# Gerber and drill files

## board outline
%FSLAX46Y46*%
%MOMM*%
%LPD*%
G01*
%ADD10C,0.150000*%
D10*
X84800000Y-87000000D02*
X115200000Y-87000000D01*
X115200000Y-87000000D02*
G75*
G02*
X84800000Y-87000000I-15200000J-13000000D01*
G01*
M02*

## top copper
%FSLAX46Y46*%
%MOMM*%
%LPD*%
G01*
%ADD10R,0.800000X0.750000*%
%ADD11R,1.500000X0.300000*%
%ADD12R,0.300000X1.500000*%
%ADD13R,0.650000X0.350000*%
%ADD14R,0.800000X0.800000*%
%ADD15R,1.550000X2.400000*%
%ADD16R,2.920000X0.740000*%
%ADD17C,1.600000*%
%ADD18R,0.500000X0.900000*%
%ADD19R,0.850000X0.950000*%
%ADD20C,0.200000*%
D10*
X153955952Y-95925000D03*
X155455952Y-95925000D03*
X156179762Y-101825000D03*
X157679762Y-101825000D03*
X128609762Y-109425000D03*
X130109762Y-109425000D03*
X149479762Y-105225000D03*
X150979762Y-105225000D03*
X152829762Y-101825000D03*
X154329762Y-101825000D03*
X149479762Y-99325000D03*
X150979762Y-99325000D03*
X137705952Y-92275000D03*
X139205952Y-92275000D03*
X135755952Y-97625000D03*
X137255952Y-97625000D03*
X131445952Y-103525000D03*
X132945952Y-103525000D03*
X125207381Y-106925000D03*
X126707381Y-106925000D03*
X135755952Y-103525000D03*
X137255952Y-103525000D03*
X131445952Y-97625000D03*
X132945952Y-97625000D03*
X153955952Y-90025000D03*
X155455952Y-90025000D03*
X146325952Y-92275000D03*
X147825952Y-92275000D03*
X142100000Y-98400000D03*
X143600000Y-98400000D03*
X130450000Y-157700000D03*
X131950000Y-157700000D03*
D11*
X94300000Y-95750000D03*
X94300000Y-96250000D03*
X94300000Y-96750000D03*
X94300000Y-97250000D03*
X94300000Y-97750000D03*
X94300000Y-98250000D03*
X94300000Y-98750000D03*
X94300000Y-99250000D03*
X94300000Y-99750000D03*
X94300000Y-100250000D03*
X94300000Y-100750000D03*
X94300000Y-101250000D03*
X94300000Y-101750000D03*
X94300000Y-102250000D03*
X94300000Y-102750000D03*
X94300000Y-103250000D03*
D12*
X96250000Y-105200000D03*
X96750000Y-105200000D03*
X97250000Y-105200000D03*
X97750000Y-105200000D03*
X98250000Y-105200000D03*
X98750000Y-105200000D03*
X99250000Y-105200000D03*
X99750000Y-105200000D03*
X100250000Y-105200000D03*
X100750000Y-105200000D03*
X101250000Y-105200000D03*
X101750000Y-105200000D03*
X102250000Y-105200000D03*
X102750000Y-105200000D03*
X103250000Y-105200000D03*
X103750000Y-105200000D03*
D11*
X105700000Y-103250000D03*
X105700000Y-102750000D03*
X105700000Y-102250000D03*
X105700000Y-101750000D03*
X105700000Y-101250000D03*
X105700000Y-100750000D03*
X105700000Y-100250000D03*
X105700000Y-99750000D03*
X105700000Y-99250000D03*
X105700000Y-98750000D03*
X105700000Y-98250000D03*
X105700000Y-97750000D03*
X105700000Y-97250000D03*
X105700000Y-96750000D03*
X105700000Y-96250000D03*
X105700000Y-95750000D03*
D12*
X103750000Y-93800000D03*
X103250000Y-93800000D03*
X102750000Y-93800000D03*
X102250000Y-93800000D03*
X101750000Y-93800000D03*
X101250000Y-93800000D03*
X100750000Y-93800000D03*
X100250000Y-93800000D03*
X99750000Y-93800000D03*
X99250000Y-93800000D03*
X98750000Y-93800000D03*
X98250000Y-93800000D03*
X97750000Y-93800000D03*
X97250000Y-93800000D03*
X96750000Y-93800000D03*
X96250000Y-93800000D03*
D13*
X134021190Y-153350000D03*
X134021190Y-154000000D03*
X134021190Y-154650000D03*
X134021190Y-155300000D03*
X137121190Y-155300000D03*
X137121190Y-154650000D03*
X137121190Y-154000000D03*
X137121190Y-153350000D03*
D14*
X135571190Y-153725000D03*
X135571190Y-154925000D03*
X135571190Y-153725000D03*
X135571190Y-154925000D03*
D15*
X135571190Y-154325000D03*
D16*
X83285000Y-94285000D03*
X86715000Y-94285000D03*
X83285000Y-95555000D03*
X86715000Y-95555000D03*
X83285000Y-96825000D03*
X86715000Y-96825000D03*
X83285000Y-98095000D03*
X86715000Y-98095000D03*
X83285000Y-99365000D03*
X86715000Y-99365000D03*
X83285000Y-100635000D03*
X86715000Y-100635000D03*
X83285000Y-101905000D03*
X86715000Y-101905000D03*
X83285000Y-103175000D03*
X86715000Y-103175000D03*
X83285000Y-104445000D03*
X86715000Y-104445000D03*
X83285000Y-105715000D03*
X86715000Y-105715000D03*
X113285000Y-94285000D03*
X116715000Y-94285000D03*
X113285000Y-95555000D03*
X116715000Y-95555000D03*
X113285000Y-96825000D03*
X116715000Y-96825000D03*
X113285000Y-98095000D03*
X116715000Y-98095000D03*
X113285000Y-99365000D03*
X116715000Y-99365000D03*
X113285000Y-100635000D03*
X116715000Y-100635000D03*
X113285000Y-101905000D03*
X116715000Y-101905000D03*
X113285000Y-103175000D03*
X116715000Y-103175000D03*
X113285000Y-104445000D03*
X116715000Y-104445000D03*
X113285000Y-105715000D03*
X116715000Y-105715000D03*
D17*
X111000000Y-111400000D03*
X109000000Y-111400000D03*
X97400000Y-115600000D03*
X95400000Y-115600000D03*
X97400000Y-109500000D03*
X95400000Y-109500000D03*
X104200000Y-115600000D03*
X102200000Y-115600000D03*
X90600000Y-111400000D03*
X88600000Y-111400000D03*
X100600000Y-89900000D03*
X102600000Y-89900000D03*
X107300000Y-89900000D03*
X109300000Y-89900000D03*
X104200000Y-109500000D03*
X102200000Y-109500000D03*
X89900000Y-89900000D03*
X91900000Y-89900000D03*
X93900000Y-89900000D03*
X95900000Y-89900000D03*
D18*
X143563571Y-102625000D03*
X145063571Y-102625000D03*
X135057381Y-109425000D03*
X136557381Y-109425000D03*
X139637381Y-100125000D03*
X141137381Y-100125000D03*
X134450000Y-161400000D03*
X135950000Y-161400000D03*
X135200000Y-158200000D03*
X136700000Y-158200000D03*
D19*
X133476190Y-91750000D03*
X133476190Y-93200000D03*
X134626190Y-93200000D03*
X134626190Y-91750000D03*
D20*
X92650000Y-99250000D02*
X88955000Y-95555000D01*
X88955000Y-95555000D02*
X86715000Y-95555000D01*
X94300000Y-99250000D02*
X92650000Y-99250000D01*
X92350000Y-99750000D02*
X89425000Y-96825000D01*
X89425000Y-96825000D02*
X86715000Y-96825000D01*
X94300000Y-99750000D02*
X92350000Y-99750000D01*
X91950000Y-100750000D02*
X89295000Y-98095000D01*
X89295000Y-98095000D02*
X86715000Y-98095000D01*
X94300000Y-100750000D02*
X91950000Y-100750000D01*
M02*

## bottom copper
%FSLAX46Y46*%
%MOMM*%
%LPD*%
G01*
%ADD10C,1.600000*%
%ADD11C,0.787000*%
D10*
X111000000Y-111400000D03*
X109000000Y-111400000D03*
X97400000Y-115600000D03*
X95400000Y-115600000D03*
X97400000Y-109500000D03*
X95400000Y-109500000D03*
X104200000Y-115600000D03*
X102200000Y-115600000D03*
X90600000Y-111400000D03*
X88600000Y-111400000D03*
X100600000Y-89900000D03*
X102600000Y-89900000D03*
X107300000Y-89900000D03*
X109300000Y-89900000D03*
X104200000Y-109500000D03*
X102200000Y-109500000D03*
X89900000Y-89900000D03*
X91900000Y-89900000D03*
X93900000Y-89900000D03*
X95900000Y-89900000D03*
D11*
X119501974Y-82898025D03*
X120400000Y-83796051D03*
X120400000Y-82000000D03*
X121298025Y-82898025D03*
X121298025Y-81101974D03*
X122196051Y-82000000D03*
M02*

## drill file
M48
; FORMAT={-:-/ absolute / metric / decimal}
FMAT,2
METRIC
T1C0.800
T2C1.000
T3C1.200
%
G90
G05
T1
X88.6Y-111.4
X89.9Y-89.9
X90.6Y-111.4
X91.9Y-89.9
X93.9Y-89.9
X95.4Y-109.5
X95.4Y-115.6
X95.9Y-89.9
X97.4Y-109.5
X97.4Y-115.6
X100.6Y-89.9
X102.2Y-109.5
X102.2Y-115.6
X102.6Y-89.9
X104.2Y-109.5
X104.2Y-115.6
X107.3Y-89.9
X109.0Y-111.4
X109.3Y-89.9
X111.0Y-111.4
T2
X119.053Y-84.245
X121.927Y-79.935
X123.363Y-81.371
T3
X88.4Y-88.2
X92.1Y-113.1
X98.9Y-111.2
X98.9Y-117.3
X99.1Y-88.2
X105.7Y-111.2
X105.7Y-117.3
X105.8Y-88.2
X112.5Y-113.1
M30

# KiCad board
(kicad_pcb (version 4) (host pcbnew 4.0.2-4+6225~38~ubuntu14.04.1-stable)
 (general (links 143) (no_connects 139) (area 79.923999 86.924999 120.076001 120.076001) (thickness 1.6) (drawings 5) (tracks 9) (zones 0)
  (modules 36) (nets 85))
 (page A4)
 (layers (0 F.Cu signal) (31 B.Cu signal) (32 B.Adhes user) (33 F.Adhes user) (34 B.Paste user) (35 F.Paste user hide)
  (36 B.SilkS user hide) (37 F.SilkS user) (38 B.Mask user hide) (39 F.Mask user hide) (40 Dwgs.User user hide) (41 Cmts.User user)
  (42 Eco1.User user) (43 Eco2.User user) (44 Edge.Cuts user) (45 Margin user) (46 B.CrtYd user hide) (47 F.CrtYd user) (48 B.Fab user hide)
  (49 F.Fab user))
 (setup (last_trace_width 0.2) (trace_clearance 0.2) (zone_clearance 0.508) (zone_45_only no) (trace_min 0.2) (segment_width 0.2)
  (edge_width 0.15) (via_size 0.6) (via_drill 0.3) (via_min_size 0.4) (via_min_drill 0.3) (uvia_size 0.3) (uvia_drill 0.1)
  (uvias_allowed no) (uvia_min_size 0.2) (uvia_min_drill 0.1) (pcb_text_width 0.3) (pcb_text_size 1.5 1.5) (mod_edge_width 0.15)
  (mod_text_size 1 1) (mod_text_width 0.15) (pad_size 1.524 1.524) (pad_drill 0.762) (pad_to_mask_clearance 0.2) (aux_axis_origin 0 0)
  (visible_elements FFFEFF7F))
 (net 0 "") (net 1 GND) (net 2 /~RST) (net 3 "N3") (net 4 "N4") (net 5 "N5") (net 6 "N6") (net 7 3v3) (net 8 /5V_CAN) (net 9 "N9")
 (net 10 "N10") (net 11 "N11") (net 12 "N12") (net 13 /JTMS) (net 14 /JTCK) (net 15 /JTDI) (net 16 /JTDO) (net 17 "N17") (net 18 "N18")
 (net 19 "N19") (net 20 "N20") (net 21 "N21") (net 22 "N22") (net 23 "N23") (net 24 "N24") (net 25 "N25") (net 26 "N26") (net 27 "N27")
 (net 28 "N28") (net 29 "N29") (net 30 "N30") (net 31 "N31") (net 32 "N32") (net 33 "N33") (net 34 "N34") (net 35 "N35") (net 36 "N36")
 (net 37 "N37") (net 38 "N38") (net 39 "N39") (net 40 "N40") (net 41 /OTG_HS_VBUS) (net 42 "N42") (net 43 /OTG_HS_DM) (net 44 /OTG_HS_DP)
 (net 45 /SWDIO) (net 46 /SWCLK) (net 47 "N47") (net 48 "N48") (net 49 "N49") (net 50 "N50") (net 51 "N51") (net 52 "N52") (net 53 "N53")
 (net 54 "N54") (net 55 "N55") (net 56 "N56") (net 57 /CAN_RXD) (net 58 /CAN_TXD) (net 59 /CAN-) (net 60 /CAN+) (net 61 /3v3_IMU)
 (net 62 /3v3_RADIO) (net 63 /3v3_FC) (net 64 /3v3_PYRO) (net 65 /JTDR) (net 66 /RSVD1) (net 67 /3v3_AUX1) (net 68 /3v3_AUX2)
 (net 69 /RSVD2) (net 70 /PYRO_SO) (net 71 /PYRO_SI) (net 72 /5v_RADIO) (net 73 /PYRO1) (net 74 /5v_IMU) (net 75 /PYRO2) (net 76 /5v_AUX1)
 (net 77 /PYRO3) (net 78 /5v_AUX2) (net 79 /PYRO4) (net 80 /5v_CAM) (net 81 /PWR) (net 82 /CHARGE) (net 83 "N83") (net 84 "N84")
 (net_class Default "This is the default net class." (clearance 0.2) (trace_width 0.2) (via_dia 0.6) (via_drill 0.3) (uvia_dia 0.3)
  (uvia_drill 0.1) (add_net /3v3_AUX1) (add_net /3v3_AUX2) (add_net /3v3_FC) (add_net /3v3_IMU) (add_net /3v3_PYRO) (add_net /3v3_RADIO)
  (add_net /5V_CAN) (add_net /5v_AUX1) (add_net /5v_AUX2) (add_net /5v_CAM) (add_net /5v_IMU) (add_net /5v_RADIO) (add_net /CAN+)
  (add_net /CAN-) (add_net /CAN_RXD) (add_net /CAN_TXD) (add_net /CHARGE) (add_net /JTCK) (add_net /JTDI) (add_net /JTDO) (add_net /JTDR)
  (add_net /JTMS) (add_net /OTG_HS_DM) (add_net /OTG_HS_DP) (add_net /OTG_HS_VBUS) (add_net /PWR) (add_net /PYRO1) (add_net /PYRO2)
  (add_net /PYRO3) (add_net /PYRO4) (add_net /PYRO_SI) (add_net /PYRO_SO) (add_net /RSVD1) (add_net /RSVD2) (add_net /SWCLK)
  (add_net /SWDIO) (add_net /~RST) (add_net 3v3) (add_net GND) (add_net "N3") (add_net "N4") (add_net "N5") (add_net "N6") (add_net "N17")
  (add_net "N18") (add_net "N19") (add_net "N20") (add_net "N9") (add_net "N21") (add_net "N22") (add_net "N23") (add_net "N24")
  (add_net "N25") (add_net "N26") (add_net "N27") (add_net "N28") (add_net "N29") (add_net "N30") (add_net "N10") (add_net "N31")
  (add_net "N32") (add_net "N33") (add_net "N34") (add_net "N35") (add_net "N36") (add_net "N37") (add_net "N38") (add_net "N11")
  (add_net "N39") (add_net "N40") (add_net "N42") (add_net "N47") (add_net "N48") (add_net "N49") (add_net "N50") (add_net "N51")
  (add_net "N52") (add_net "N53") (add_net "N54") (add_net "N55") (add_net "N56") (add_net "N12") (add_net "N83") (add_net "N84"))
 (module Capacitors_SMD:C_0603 (layer F.Cu) (at 154.705952 95.925)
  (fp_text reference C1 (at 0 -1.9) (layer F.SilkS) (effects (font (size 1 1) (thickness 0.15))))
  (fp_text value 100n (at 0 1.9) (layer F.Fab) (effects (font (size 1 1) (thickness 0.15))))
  (pad 1 smd rect (at -0.75 0) (size 0.8 0.75) (layers F.Cu F.Paste F.Mask) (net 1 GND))
  (pad 2 smd rect (at 0.75 0) (size 0.8 0.75) (layers F.Cu F.Paste F.Mask) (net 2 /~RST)))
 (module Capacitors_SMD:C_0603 (layer F.Cu) (at 156.929762 101.825)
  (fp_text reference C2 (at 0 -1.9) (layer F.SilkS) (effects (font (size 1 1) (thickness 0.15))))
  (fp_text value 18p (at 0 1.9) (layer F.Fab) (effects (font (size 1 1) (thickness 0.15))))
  (pad 1 smd rect (at -0.75 0) (size 0.8 0.75) (layers F.Cu F.Paste F.Mask) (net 1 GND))
  (pad 2 smd rect (at 0.75 0) (size 0.8 0.75) (layers F.Cu F.Paste F.Mask) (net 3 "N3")))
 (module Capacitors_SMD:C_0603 (layer F.Cu) (at 129.359762 109.425)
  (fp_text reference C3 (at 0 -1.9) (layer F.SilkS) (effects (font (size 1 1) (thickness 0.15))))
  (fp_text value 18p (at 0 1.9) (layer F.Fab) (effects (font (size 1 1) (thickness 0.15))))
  (pad 1 smd rect (at -0.75 0) (size 0.8 0.75) (layers F.Cu F.Paste F.Mask) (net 1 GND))
  (pad 2 smd rect (at 0.75 0) (size 0.8 0.75) (layers F.Cu F.Paste F.Mask) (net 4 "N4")))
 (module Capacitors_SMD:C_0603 (layer F.Cu) (at 150.229762 105.225)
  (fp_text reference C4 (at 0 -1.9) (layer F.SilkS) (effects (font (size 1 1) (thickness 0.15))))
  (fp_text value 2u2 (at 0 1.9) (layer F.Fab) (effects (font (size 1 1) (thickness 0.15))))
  (pad 1 smd rect (at -0.75 0) (size 0.8 0.75) (layers F.Cu F.Paste F.Mask) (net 1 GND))
  (pad 2 smd rect (at 0.75 0) (size 0.8 0.75) (layers F.Cu F.Paste F.Mask) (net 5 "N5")))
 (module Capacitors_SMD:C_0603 (layer F.Cu) (at 153.579762 101.825)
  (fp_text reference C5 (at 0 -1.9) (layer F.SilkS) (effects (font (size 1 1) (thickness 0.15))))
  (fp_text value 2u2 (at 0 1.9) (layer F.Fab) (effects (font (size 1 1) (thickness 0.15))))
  (pad 1 smd rect (at -0.75 0) (size 0.8 0.75) (layers F.Cu F.Paste F.Mask) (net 1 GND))
  (pad 2 smd rect (at 0.75 0) (size 0.8 0.75) (layers F.Cu F.Paste F.Mask) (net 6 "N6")))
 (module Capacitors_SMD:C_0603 (layer F.Cu) (at 150.229762 99.325)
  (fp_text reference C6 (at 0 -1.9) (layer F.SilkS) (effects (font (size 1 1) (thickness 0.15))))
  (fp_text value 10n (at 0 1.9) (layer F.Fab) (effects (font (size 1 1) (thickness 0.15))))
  (pad 1 smd rect (at -0.75 0) (size 0.8 0.75) (layers F.Cu F.Paste F.Mask) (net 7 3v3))
  (pad 2 smd rect (at 0.75 0) (size 0.8 0.75) (layers F.Cu F.Paste F.Mask) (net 1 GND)))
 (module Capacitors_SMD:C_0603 (layer F.Cu) (at 138.455952 92.275)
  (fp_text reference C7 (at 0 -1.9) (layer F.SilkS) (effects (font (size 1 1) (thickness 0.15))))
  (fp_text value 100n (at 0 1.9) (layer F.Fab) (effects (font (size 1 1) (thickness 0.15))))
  (pad 1 smd rect (at -0.75 0) (size 0.8 0.75) (layers F.Cu F.Paste F.Mask) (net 7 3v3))
  (pad 2 smd rect (at 0.75 0) (size 0.8 0.75) (layers F.Cu F.Paste F.Mask) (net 1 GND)))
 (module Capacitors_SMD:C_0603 (layer F.Cu) (at 136.505952 97.625)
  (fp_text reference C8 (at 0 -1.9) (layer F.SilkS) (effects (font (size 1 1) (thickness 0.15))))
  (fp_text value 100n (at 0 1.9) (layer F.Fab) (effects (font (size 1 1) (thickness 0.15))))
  (pad 1 smd rect (at -0.75 0) (size 0.8 0.75) (layers F.Cu F.Paste F.Mask) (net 7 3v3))
  (pad 2 smd rect (at 0.75 0) (size 0.8 0.75) (layers F.Cu F.Paste F.Mask) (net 1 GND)))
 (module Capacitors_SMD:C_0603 (layer F.Cu) (at 132.195952 103.525)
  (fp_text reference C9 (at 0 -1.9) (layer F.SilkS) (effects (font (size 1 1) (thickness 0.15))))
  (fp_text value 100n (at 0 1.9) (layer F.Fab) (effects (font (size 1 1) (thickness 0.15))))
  (pad 1 smd rect (at -0.75 0) (size 0.8 0.75) (layers F.Cu F.Paste F.Mask) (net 7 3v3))
  (pad 2 smd rect (at 0.75 0) (size 0.8 0.75) (layers F.Cu F.Paste F.Mask) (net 1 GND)))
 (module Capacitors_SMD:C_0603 (layer F.Cu) (at 125.957381 106.925)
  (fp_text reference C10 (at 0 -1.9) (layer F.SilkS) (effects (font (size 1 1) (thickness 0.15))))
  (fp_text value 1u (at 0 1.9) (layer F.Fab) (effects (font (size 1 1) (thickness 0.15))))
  (pad 1 smd rect (at -0.75 0) (size 0.8 0.75) (layers F.Cu F.Paste F.Mask) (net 7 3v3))
  (pad 2 smd rect (at 0.75 0) (size 0.8 0.75) (layers F.Cu F.Paste F.Mask) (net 1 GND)))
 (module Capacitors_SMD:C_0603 (layer F.Cu) (at 136.505952 103.525)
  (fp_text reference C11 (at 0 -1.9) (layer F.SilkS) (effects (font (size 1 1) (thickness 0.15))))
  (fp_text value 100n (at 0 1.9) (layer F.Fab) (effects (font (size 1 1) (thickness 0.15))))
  (pad 1 smd rect (at -0.75 0) (size 0.8 0.75) (layers F.Cu F.Paste F.Mask) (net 7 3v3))
  (pad 2 smd rect (at 0.75 0) (size 0.8 0.75) (layers F.Cu F.Paste F.Mask) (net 1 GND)))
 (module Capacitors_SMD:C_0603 (layer F.Cu) (at 132.195952 97.625)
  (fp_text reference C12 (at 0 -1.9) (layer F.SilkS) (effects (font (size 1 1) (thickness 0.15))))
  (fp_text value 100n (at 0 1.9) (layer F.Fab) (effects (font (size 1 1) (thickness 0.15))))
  (pad 1 smd rect (at -0.75 0) (size 0.8 0.75) (layers F.Cu F.Paste F.Mask) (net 7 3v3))
  (pad 2 smd rect (at 0.75 0) (size 0.8 0.75) (layers F.Cu F.Paste F.Mask) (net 1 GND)))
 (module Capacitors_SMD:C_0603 (layer F.Cu) (at 154.705952 90.025)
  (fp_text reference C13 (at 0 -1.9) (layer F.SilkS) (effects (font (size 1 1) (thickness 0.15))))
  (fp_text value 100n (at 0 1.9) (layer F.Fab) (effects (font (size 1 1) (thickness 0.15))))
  (pad 1 smd rect (at -0.75 0) (size 0.8 0.75) (layers F.Cu F.Paste F.Mask) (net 7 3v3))
  (pad 2 smd rect (at 0.75 0) (size 0.8 0.75) (layers F.Cu F.Paste F.Mask) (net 1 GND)))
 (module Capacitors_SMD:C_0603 (layer F.Cu) (at 147.075952 92.275)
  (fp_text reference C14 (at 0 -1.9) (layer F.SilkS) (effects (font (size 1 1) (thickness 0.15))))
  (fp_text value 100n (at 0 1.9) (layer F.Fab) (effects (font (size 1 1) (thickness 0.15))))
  (pad 1 smd rect (at -0.75 0) (size 0.8 0.75) (layers F.Cu F.Paste F.Mask) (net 7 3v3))
  (pad 2 smd rect (at 0.75 0) (size 0.8 0.75) (layers F.Cu F.Paste F.Mask) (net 1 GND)))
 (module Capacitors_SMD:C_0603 (layer F.Cu) (at 142.85 98.4)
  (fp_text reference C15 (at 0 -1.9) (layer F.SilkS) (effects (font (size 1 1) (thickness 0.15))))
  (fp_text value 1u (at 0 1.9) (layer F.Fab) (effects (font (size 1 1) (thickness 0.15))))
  (pad 1 smd rect (at -0.75 0) (size 0.8 0.75) (layers F.Cu F.Paste F.Mask) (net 7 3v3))
  (pad 2 smd rect (at 0.75 0) (size 0.8 0.75) (layers F.Cu F.Paste F.Mask) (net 1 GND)))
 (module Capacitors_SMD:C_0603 (layer F.Cu) (at 131.2 157.7)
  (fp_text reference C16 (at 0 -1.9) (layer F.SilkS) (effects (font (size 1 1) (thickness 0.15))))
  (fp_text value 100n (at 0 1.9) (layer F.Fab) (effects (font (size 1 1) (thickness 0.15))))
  (pad 1 smd rect (at -0.75 0) (size 0.8 0.75) (layers F.Cu F.Paste F.Mask) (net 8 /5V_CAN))
  (pad 2 smd rect (at 0.75 0) (size 0.8 0.75) (layers F.Cu F.Paste F.Mask) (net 1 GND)))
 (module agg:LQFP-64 (layer F.Cu) (at 100 99.5)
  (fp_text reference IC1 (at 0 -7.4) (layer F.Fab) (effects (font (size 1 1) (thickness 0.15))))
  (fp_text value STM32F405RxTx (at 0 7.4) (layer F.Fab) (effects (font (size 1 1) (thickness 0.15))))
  (pad 1 smd rect (at -5.7 -3.75) (size 1.5 0.3) (layers F.Cu F.Paste F.Mask) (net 7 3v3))
  (pad 2 smd rect (at -5.7 -3.25) (size 1.5 0.3) (layers F.Cu F.Paste F.Mask) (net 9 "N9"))
  (pad 3 smd rect (at -5.7 -2.75) (size 1.5 0.3) (layers F.Cu F.Paste F.Mask) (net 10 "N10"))
  (pad 4 smd rect (at -5.7 -2.25) (size 1.5 0.3) (layers F.Cu F.Paste F.Mask) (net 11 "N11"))
  (pad 5 smd rect (at -5.7 -1.75) (size 1.5 0.3) (layers F.Cu F.Paste F.Mask) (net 3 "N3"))
  (pad 6 smd rect (at -5.7 -1.25) (size 1.5 0.3) (layers F.Cu F.Paste F.Mask) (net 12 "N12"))
  (pad 7 smd rect (at -5.7 -0.75) (size 1.5 0.3) (layers F.Cu F.Paste F.Mask) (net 2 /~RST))
  (pad 8 smd rect (at -5.7 -0.25) (size 1.5 0.3) (layers F.Cu F.Paste F.Mask) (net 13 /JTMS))
  (pad 9 smd rect (at -5.7 0.25) (size 1.5 0.3) (layers F.Cu F.Paste F.Mask) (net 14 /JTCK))
  (pad 10 smd rect (at -5.7 0.75) (size 1.5 0.3) (layers F.Cu F.Paste F.Mask) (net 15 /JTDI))
  (pad 11 smd rect (at -5.7 1.25) (size 1.5 0.3) (layers F.Cu F.Paste F.Mask) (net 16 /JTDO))
  (pad 12 smd rect (at -5.7 1.75) (size 1.5 0.3) (layers F.Cu F.Paste F.Mask) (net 1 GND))
  (pad 13 smd rect (at -5.7 2.25) (size 1.5 0.3) (layers F.Cu F.Paste F.Mask) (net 7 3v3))
  (pad 14 smd rect (at -5.7 2.75) (size 1.5 0.3) (layers F.Cu F.Paste F.Mask) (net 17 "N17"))
  (pad 15 smd rect (at -5.7 3.25) (size 1.5 0.3) (layers F.Cu F.Paste F.Mask) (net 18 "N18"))
  (pad 16 smd rect (at -5.7 3.75) (size 1.5 0.3) (layers F.Cu F.Paste F.Mask) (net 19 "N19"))
  (pad 17 smd rect (at -3.75 5.7) (size 0.3 1.5) (layers F.Cu F.Paste F.Mask) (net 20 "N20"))
  (pad 18 smd rect (at -3.25 5.7) (size 0.3 1.5) (layers F.Cu F.Paste F.Mask) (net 1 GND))
  (pad 19 smd rect (at -2.75 5.7) (size 0.3 1.5) (layers F.Cu F.Paste F.Mask) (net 7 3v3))
  (pad 20 smd rect (at -2.25 5.7) (size 0.3 1.5) (layers F.Cu F.Paste F.Mask) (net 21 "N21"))
  (pad 21 smd rect (at -1.75 5.7) (size 0.3 1.5) (layers F.Cu F.Paste F.Mask) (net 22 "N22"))
  (pad 22 smd rect (at -1.25 5.7) (size 0.3 1.5) (layers F.Cu F.Paste F.Mask) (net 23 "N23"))
  (pad 23 smd rect (at -0.75 5.7) (size 0.3 1.5) (layers F.Cu F.Paste F.Mask) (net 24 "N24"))
  (pad 24 smd rect (at -0.25 5.7) (size 0.3 1.5) (layers F.Cu F.Paste F.Mask) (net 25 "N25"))
  (pad 25 smd rect (at 0.25 5.7) (size 0.3 1.5) (layers F.Cu F.Paste F.Mask) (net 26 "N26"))
  (pad 26 smd rect (at 0.75 5.7) (size 0.3 1.5) (layers F.Cu F.Paste F.Mask) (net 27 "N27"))
  (pad 27 smd rect (at 1.25 5.7) (size 0.3 1.5) (layers F.Cu F.Paste F.Mask) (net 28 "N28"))
  (pad 28 smd rect (at 1.75 5.7) (size 0.3 1.5) (layers F.Cu F.Paste F.Mask) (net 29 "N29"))
  (pad 29 smd rect (at 2.25 5.7) (size 0.3 1.5) (layers F.Cu F.Paste F.Mask) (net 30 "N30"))
  (pad 30 smd rect (at 2.75 5.7) (size 0.3 1.5) (layers F.Cu F.Paste F.Mask) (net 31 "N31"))
  (pad 31 smd rect (at 3.25 5.7) (size 0.3 1.5) (layers F.Cu F.Paste F.Mask) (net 5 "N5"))
  (pad 32 smd rect (at 3.75 5.7) (size 0.3 1.5) (layers F.Cu F.Paste F.Mask) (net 7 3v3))
  (pad 33 smd rect (at 5.7 3.75) (size 1.5 0.3) (layers F.Cu F.Paste F.Mask) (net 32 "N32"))
  (pad 34 smd rect (at 5.7 3.25) (size 1.5 0.3) (layers F.Cu F.Paste F.Mask) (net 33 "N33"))
  (pad 35 smd rect (at 5.7 2.75) (size 1.5 0.3) (layers F.Cu F.Paste F.Mask) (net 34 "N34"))
  (pad 36 smd rect (at 5.7 2.25) (size 1.5 0.3) (layers F.Cu F.Paste F.Mask) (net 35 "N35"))
  (pad 37 smd rect (at 5.7 1.75) (size 1.5 0.3) (layers F.Cu F.Paste F.Mask) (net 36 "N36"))
  (pad 38 smd rect (at 5.7 1.25) (size 1.5 0.3) (layers F.Cu F.Paste F.Mask) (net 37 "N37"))
  (pad 39 smd rect (at 5.7 0.75) (size 1.5 0.3) (layers F.Cu F.Paste F.Mask) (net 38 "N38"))
  (pad 40 smd rect (at 5.7 0.25) (size 1.5 0.3) (layers F.Cu F.Paste F.Mask) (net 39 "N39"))
  (pad 41 smd rect (at 5.7 -0.25) (size 1.5 0.3) (layers F.Cu F.Paste F.Mask) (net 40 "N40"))
  (pad 42 smd rect (at 5.7 -0.75) (size 1.5 0.3) (layers F.Cu F.Paste F.Mask) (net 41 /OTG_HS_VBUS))
  (pad 43 smd rect (at 5.7 -1.25) (size 1.5 0.3) (layers F.Cu F.Paste F.Mask) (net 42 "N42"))
  (pad 44 smd rect (at 5.7 -1.75) (size 1.5 0.3) (layers F.Cu F.Paste F.Mask) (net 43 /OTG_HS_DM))
  (pad 45 smd rect (at 5.7 -2.25) (size 1.5 0.3) (layers F.Cu F.Paste F.Mask) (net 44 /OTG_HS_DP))
  (pad 46 smd rect (at 5.7 -2.75) (size 1.5 0.3) (layers F.Cu F.Paste F.Mask) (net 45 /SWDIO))
  (pad 47 smd rect (at 5.7 -3.25) (size 1.5 0.3) (layers F.Cu F.Paste F.Mask) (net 6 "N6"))
  (pad 48 smd rect (at 5.7 -3.75) (size 1.5 0.3) (layers F.Cu F.Paste F.Mask) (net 7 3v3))
  (pad 49 smd rect (at 3.75 -5.7) (size 0.3 1.5) (layers F.Cu F.Paste F.Mask) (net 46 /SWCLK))
  (pad 50 smd rect (at 3.25 -5.7) (size 0.3 1.5) (layers F.Cu F.Paste F.Mask) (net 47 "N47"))
  (pad 51 smd rect (at 2.75 -5.7) (size 0.3 1.5) (layers F.Cu F.Paste F.Mask) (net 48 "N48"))
  (pad 52 smd rect (at 2.25 -5.7) (size 0.3 1.5) (layers F.Cu F.Paste F.Mask) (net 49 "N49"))
  (pad 53 smd rect (at 1.75 -5.7) (size 0.3 1.5) (layers F.Cu F.Paste F.Mask) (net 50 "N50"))
  (pad 54 smd rect (at 1.25 -5.7) (size 0.3 1.5) (layers F.Cu F.Paste F.Mask) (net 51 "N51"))
  (pad 55 smd rect (at 0.75 -5.7) (size 0.3 1.5) (layers F.Cu F.Paste F.Mask) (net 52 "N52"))
  (pad 56 smd rect (at 0.25 -5.7) (size 0.3 1.5) (layers F.Cu F.Paste F.Mask) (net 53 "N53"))
  (pad 57 smd rect (at -0.25 -5.7) (size 0.3 1.5) (layers F.Cu F.Paste F.Mask) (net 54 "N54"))
  (pad 58 smd rect (at -0.75 -5.7) (size 0.3 1.5) (layers F.Cu F.Paste F.Mask) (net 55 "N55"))
  (pad 59 smd rect (at -1.25 -5.7) (size 0.3 1.5) (layers F.Cu F.Paste F.Mask) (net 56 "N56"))
  (pad 60 smd rect (at -1.75 -5.7) (size 0.3 1.5) (layers F.Cu F.Paste F.Mask) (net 1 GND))
  (pad 61 smd rect (at -2.25 -5.7) (size 0.3 1.5) (layers F.Cu F.Paste F.Mask) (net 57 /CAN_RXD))
  (pad 62 smd rect (at -2.75 -5.7) (size 0.3 1.5) (layers F.Cu F.Paste F.Mask) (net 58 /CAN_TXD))
  (pad 63 smd rect (at -3.25 -5.7) (size 0.3 1.5) (layers F.Cu F.Paste F.Mask) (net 1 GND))
  (pad 64 smd rect (at -3.75 -5.7) (size 0.3 1.5) (layers F.Cu F.Paste F.Mask) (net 7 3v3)))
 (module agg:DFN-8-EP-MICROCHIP (layer F.Cu) (at 135.57119 154.325)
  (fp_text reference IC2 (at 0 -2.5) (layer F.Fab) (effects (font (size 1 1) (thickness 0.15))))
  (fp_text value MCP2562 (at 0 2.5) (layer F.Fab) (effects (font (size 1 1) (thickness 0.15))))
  (pad 1 smd rect (at -1.55 -0.975) (size 0.65 0.35) (layers F.Cu F.Paste F.Mask) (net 58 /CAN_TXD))
  (pad 2 smd rect (at -1.55 -0.325) (size 0.65 0.35) (layers F.Cu F.Paste F.Mask) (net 1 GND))
  (pad 3 smd rect (at -1.55 0.325) (size 0.65 0.35) (layers F.Cu F.Paste F.Mask) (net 8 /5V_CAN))
  (pad 4 smd rect (at -1.55 0.975) (size 0.65 0.35) (layers F.Cu F.Paste F.Mask) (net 57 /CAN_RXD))
  (pad 5 smd rect (at 1.55 0.975) (size 0.65 0.35) (layers F.Cu F.Paste F.Mask) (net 7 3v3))
  (pad 6 smd rect (at 1.55 0.325) (size 0.65 0.35) (layers F.Cu F.Paste F.Mask) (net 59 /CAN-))
  (pad 7 smd rect (at 1.55 -0.325) (size 0.65 0.35) (layers F.Cu F.Paste F.Mask) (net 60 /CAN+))
  (pad 8 smd rect (at 1.55 -0.975) (size 0.65 0.35) (layers F.Cu F.Paste F.Mask) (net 1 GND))
  (pad EP smd rect (at 0 -0.6) (size 0.8 0.8) (layers F.Cu F.Mask) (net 1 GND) (solder_mask_margin 0.001))
  (pad EP smd rect (at 0 0.6) (size 0.8 0.8) (layers F.Cu F.Mask) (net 1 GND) (solder_mask_margin 0.001))
  (pad EP smd rect (at 0 -0.6) (size 0.8 0.8) (layers F.Cu F.Paste) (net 1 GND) (solder_paste_margin 0.001))
  (pad EP smd rect (at 0 0.6) (size 0.8 0.8) (layers F.Cu F.Paste) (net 1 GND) (solder_paste_margin 0.001))
  (pad EP smd rect (at 0 0) (size 1.55 2.4) (layers F.Cu) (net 1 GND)))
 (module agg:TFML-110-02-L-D (layer F.Cu) (at 85 100 270)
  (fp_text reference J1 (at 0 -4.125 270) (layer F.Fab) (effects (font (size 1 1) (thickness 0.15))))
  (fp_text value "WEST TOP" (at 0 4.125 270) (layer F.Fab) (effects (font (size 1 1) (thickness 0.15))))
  (pad 1 smd rect (at -5.715 1.715 270) (size 0.74 2.92) (layers F.Cu F.Paste F.Mask) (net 1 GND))
  (pad 2 smd rect (at -5.715 -1.715 270) (size 0.74 2.92) (layers F.Cu F.Paste F.Mask) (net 1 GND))
  (pad 3 smd rect (at -4.445 1.715 270) (size 0.74 2.92) (layers F.Cu F.Paste F.Mask) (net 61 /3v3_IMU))
  (pad 4 smd rect (at -4.445 -1.715 270) (size 0.74 2.92) (layers F.Cu F.Paste F.Mask) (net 13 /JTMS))
  (pad 5 smd rect (at -3.175 1.715 270) (size 0.74 2.92) (layers F.Cu F.Paste F.Mask) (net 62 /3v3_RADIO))
  (pad 6 smd rect (at -3.175 -1.715 270) (size 0.74 2.92) (layers F.Cu F.Paste F.Mask) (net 14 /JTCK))
  (pad 7 smd rect (at -1.905 1.715 270) (size 0.74 2.92) (layers F.Cu F.Paste F.Mask) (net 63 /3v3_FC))
  (pad 8 smd rect (at -1.905 -1.715 270) (size 0.74 2.92) (layers F.Cu F.Paste F.Mask) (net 16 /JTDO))
  (pad 9 smd rect (at -0.635 1.715 270) (size 0.74 2.92) (layers F.Cu F.Paste F.Mask) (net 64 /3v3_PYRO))
  (pad 10 smd rect (at -0.635 -1.715 270) (size 0.74 2.92) (layers F.Cu F.Paste F.Mask) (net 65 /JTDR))
  (pad 11 smd rect (at 0.635 1.715 270) (size 0.74 2.92) (layers F.Cu F.Paste F.Mask) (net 7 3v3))
  (pad 12 smd rect (at 0.635 -1.715 270) (size 0.74 2.92) (layers F.Cu F.Paste F.Mask) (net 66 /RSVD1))
  (pad 13 smd rect (at 1.905 1.715 270) (size 0.74 2.92) (layers F.Cu F.Paste F.Mask) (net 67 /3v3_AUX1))
  (pad 14 smd rect (at 1.905 -1.715 270) (size 0.74 2.92) (layers F.Cu F.Paste F.Mask) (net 8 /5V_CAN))
  (pad 15 smd rect (at 3.175 1.715 270) (size 0.74 2.92) (layers F.Cu F.Paste F.Mask) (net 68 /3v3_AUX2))
  (pad 16 smd rect (at 3.175 -1.715 270) (size 0.74 2.92) (layers F.Cu F.Paste F.Mask) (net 59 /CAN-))
  (pad 17 smd rect (at 4.445 1.715 270) (size 0.74 2.92) (layers F.Cu F.Paste F.Mask) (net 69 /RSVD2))
  (pad 18 smd rect (at 4.445 -1.715 270) (size 0.74 2.92) (layers F.Cu F.Paste F.Mask) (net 60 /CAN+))
  (pad 19 smd rect (at 5.715 1.715 270) (size 0.74 2.92) (layers F.Cu F.Paste F.Mask) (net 1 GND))
  (pad 20 smd rect (at 5.715 -1.715 270) (size 0.74 2.92) (layers F.Cu F.Paste F.Mask) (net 1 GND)))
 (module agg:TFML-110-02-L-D (layer F.Cu) (at 115 100 270)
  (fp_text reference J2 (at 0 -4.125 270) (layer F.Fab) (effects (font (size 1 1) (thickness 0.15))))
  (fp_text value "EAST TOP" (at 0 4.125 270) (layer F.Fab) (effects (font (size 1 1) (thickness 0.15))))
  (pad 1 smd rect (at -5.715 1.715 270) (size 0.74 2.92) (layers F.Cu F.Paste F.Mask) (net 1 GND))
  (pad 2 smd rect (at -5.715 -1.715 270) (size 0.74 2.92) (layers F.Cu F.Paste F.Mask) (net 1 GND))
  (pad 3 smd rect (at -4.445 1.715 270) (size 0.74 2.92) (layers F.Cu F.Paste F.Mask) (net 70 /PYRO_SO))
  (pad 4 smd rect (at -4.445 -1.715 270) (size 0.74 2.92) (layers F.Cu F.Paste F.Mask) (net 70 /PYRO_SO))
  (pad 5 smd rect (at -3.175 1.715 270) (size 0.74 2.92) (layers F.Cu F.Paste F.Mask) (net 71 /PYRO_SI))
  (pad 6 smd rect (at -3.175 -1.715 270) (size 0.74 2.92) (layers F.Cu F.Paste F.Mask) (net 71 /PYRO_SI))
  (pad 7 smd rect (at -1.905 1.715 270) (size 0.74 2.92) (layers F.Cu F.Paste F.Mask) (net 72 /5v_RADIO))
  (pad 8 smd rect (at -1.905 -1.715 270) (size 0.74 2.92) (layers F.Cu F.Paste F.Mask) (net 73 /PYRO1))
  (pad 9 smd rect (at -0.635 1.715 270) (size 0.74 2.92) (layers F.Cu F.Paste F.Mask) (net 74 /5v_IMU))
  (pad 10 smd rect (at -0.635 -1.715 270) (size 0.74 2.92) (layers F.Cu F.Paste F.Mask) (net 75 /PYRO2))
  (pad 11 smd rect (at 0.635 1.715 270) (size 0.74 2.92) (layers F.Cu F.Paste F.Mask) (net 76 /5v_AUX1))
  (pad 12 smd rect (at 0.635 -1.715 270) (size 0.74 2.92) (layers F.Cu F.Paste F.Mask) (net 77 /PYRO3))
  (pad 13 smd rect (at 1.905 1.715 270) (size 0.74 2.92) (layers F.Cu F.Paste F.Mask) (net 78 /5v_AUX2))
  (pad 14 smd rect (at 1.905 -1.715 270) (size 0.74 2.92) (layers F.Cu F.Paste F.Mask) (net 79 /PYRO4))
  (pad 15 smd rect (at 3.175 1.715 270) (size 0.74 2.92) (layers F.Cu F.Paste F.Mask) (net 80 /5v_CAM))
  (pad 16 smd rect (at 3.175 -1.715 270) (size 0.74 2.92) (layers F.Cu F.Paste F.Mask) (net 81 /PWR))
  (pad 17 smd rect (at 4.445 1.715 270) (size 0.74 2.92) (layers F.Cu F.Paste F.Mask) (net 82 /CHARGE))
  (pad 18 smd rect (at 4.445 -1.715 270) (size 0.74 2.92) (layers F.Cu F.Paste F.Mask) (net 82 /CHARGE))
  (pad 19 smd rect (at 5.715 1.715 270) (size 0.74 2.92) (layers F.Cu F.Paste F.Mask) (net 1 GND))
  (pad 20 smd rect (at 5.715 -1.715 270) (size 0.74 2.92) (layers F.Cu F.Paste F.Mask) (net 1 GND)))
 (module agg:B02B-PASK (layer B.Cu) (at 110 111.4)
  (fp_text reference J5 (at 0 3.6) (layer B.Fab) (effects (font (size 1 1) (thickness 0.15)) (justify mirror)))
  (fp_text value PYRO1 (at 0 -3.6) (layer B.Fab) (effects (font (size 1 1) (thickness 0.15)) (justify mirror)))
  (pad "" np_thru_hole circle (at 2.5 1.7) (size 1.2 1.2) (drill 1.2) (layers *.Mask))
  (pad 1 thru_hole circle (at 1 0) (size 1.6 1.6) (drill 0.8) (layers *.Cu *.Mask) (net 73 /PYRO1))
  (pad 2 thru_hole circle (at -1 0) (size 1.6 1.6) (drill 0.8) (layers *.Cu *.Mask) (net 1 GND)))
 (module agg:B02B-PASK (layer B.Cu) (at 96.4 115.6)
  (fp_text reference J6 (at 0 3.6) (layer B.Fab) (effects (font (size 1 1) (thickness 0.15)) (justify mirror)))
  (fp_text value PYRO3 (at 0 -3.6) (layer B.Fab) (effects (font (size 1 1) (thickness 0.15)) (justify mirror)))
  (pad "" np_thru_hole circle (at 2.5 1.7) (size 1.2 1.2) (drill 1.2) (layers *.Mask))
  (pad 1 thru_hole circle (at 1 0) (size 1.6 1.6) (drill 0.8) (layers *.Cu *.Mask) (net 77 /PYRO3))
  (pad 2 thru_hole circle (at -1 0) (size 1.6 1.6) (drill 0.8) (layers *.Cu *.Mask) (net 1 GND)))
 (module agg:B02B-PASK (layer B.Cu) (at 96.4 109.5)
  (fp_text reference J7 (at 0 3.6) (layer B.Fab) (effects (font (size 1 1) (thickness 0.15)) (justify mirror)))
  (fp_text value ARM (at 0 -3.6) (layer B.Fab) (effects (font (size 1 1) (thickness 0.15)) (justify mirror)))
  (pad "" np_thru_hole circle (at 2.5 1.7) (size 1.2 1.2) (drill 1.2) (layers *.Mask))
  (pad 1 thru_hole circle (at 1 0) (size 1.6 1.6) (drill 0.8) (layers *.Cu *.Mask) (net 70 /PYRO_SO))
  (pad 2 thru_hole circle (at -1 0) (size 1.6 1.6) (drill 0.8) (layers *.Cu *.Mask) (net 71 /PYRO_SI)))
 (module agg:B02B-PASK (layer B.Cu) (at 103.2 115.6)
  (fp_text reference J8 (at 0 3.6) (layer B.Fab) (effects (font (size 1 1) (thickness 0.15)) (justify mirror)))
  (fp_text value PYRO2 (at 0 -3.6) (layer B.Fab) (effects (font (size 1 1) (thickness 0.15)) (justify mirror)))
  (pad "" np_thru_hole circle (at 2.5 1.7) (size 1.2 1.2) (drill 1.2) (layers *.Mask))
  (pad 1 thru_hole circle (at 1 0) (size 1.6 1.6) (drill 0.8) (layers *.Cu *.Mask) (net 75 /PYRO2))
  (pad 2 thru_hole circle (at -1 0) (size 1.6 1.6) (drill 0.8) (layers *.Cu *.Mask) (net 1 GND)))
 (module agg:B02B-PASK (layer B.Cu) (at 89.6 111.4)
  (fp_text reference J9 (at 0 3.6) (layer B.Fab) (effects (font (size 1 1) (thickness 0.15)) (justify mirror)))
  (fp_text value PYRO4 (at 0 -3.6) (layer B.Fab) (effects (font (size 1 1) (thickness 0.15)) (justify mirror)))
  (pad "" np_thru_hole circle (at 2.5 1.7) (size 1.2 1.2) (drill 1.2) (layers *.Mask))
  (pad 1 thru_hole circle (at 1 0) (size 1.6 1.6) (drill 0.8) (layers *.Cu *.Mask) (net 79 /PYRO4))
  (pad 2 thru_hole circle (at -1 0) (size 1.6 1.6) (drill 0.8) (layers *.Cu *.Mask) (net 1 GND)))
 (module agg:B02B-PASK (layer B.Cu) (at 101.6 89.9 180)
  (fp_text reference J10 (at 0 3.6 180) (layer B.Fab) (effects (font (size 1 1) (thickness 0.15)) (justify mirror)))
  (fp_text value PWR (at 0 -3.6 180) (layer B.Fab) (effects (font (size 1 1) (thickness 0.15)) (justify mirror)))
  (pad "" np_thru_hole circle (at 2.5 1.7 180) (size 1.2 1.2) (drill 1.2) (layers *.Mask))
  (pad 1 thru_hole circle (at 1 0 180) (size 1.6 1.6) (drill 0.8) (layers *.Cu *.Mask) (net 81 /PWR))
  (pad 2 thru_hole circle (at -1 0 180) (size 1.6 1.6) (drill 0.8) (layers *.Cu *.Mask) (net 1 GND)))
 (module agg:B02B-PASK (layer B.Cu) (at 108.3 89.9 180)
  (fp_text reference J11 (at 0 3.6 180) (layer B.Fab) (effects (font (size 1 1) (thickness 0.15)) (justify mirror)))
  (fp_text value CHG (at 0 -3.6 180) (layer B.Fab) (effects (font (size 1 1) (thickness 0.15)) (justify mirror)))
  (pad "" np_thru_hole circle (at 2.5 1.7 180) (size 1.2 1.2) (drill 1.2) (layers *.Mask))
  (pad 1 thru_hole circle (at 1 0 180) (size 1.6 1.6) (drill 0.8) (layers *.Cu *.Mask) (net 82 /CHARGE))
  (pad 2 thru_hole circle (at -1 0 180) (size 1.6 1.6) (drill 0.8) (layers *.Cu *.Mask) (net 1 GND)))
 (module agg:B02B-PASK (layer B.Cu) (at 103.2 109.5)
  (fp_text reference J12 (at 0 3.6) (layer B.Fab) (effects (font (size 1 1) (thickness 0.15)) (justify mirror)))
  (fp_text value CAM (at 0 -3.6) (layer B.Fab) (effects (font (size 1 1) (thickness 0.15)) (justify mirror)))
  (pad "" np_thru_hole circle (at 2.5 1.7) (size 1.2 1.2) (drill 1.2) (layers *.Mask))
  (pad 1 thru_hole circle (at 1 0) (size 1.6 1.6) (drill 0.8) (layers *.Cu *.Mask) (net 80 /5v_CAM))
  (pad 2 thru_hole circle (at -1 0) (size 1.6 1.6) (drill 0.8) (layers *.Cu *.Mask) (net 1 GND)))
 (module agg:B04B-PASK (layer B.Cu) (at 92.9 89.9 180)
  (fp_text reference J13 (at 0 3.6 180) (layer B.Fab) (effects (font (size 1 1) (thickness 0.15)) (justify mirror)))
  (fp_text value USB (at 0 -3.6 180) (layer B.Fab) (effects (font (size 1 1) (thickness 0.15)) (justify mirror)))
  (pad "" np_thru_hole circle (at 4.5 1.7 180) (size 1.2 1.2) (drill 1.2) (layers *.Mask))
  (pad 1 thru_hole circle (at 3 0 180) (size 1.6 1.6) (drill 0.8) (layers *.Cu *.Mask) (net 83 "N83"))
  (pad 2 thru_hole circle (at 1 0 180) (size 1.6 1.6) (drill 0.8) (layers *.Cu *.Mask) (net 43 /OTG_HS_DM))
  (pad 3 thru_hole circle (at -1 0 180) (size 1.6 1.6) (drill 0.8) (layers *.Cu *.Mask) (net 44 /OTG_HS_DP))
  (pad 4 thru_hole circle (at -3 0 180) (size 1.6 1.6) (drill 0.8) (layers *.Cu *.Mask) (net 1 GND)))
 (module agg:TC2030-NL (layer B.Cu) (at 120.852548 82.452548 45)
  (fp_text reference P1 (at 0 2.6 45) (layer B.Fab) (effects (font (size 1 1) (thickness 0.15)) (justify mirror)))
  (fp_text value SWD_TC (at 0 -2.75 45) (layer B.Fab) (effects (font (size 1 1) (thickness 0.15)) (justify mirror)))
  (pad 1 smd circle (at -1.27 -0.64 45) (size 0.787 0.787) (layers B.Cu B.Mask) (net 7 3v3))
  (pad 2 smd circle (at -1.27 0.63 45) (size 0.787 0.787) (layers B.Cu B.Mask) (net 45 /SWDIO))
  (pad 3 smd circle (at 0 -0.64 45) (size 0.787 0.787) (layers B.Cu B.Mask) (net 2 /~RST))
  (pad 4 smd circle (at 0 0.63 45) (size 0.787 0.787) (layers B.Cu B.Mask) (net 46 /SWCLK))
  (pad 5 smd circle (at 1.27 -0.64 45) (size 0.787 0.787) (layers B.Cu B.Mask) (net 1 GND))
  (pad 6 smd circle (at 1.27 0.63 45) (size 0.787 0.787) (layers B.Cu B.Mask) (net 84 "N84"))
  (pad "" np_thru_hole circle (at -2.54 -0.005 45) (size 1 1) (drill 1) (layers *.Cu *.Mask B.SilkS))
  (pad "" np_thru_hole circle (at 2.54 -1.021 45) (size 1 1) (drill 1) (layers *.Cu *.Mask B.SilkS))
  (pad "" np_thru_hole circle (at 2.54 1.011 45) (size 1 1) (drill 1) (layers *.Cu *.Mask B.SilkS)))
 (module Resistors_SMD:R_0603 (layer F.Cu) (at 144.313571 102.625)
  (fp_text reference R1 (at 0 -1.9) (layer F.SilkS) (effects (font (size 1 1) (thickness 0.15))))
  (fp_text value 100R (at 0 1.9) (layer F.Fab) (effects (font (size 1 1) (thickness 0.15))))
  (pad 1 smd rect (at -0.75 0) (size 0.5 0.9) (layers F.Cu F.Paste F.Mask) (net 4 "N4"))
  (pad 2 smd rect (at 0.75 0) (size 0.5 0.9) (layers F.Cu F.Paste F.Mask) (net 12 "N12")))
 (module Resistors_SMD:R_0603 (layer F.Cu) (at 135.807381 109.425)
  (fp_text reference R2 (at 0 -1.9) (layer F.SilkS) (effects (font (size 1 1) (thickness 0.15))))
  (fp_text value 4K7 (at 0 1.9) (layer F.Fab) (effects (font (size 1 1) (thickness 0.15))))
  (pad 1 smd rect (at -0.75 0) (size 0.5 0.9) (layers F.Cu F.Paste F.Mask) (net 27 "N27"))
  (pad 2 smd rect (at 0.75 0) (size 0.5 0.9) (layers F.Cu F.Paste F.Mask) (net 7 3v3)))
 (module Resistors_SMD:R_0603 (layer F.Cu) (at 140.387381 100.125)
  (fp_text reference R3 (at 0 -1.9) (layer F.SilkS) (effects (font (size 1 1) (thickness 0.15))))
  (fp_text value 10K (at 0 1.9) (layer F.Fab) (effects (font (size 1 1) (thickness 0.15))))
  (pad 1 smd rect (at -0.75 0) (size 0.5 0.9) (layers F.Cu F.Paste F.Mask) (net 1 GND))
  (pad 2 smd rect (at 0.75 0) (size 0.5 0.9) (layers F.Cu F.Paste F.Mask) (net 27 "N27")))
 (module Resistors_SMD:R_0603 (layer F.Cu) (at 135.2 161.4)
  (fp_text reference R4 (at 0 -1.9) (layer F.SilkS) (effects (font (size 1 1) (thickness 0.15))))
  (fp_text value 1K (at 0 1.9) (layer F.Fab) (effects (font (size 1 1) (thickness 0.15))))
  (pad 1 smd rect (at -0.75 0) (size 0.5 0.9) (layers F.Cu F.Paste F.Mask) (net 83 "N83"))
  (pad 2 smd rect (at 0.75 0) (size 0.5 0.9) (layers F.Cu F.Paste F.Mask) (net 41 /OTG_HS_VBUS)))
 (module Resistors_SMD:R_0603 (layer F.Cu) (at 135.95 158.2)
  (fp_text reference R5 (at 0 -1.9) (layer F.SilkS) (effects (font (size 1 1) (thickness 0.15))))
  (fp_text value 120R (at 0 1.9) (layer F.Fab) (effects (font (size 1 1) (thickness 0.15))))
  (pad 1 smd rect (at -0.75 0) (size 0.5 0.9) (layers F.Cu F.Paste F.Mask) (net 59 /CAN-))
  (pad 2 smd rect (at 0.75 0) (size 0.5 0.9) (layers F.Cu F.Paste F.Mask) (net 60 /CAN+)))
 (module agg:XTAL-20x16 (layer F.Cu) (at 134.05119 92.475)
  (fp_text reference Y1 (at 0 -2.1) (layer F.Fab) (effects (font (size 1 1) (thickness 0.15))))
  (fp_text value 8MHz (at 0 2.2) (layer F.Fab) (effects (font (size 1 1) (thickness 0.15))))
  (pad 1 smd rect (at -0.575 -0.725 270) (size 0.95 0.85) (layers F.Cu F.Paste F.Mask) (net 4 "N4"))
  (pad 2 smd rect (at -0.575 0.725 270) (size 0.95 0.85) (layers F.Cu F.Paste F.Mask) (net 3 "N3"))
  (pad 3 smd rect (at 0.575 0.725 270) (size 0.95 0.85) (layers F.Cu F.Paste F.Mask))
  (pad 4 smd rect (at 0.575 -0.725 270) (size 0.95 0.85) (layers F.Cu F.Paste F.Mask)))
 (gr_line (start 84.8 87) (end 115.2 87) (layer Edge.Cuts) (width 0.15))
 (gr_arc (start 100 100) (end 115.2 87) (angle 261.0783035) (layer Edge.Cuts) (width 0.15))
 (segment (start 92.65 99.25) (end 88.955 95.555) (width 0.2) (layer F.Cu) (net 13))
 (segment (start 88.955 95.555) (end 86.715 95.555) (width 0.2) (layer F.Cu) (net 13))
 (segment (start 94.3 99.25) (end 92.65 99.25) (width 0.2) (layer F.Cu) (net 13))
 (segment (start 92.35 99.75) (end 89.425 96.825) (width 0.2) (layer F.Cu) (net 14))
 (segment (start 89.425 96.825) (end 86.715 96.825) (width 0.2) (layer F.Cu) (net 14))
 (segment (start 94.3 99.75) (end 92.35 99.75) (width 0.2) (layer F.Cu) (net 14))
 (segment (start 91.95 100.75) (end 89.295 98.095) (width 0.2) (layer F.Cu) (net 16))
 (segment (start 89.295 98.095) (end 86.715 98.095) (width 0.2) (layer F.Cu) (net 16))
 (segment (start 94.3 100.75) (end 91.95 100.75) (width 0.2) (layer F.Cu) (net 16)))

